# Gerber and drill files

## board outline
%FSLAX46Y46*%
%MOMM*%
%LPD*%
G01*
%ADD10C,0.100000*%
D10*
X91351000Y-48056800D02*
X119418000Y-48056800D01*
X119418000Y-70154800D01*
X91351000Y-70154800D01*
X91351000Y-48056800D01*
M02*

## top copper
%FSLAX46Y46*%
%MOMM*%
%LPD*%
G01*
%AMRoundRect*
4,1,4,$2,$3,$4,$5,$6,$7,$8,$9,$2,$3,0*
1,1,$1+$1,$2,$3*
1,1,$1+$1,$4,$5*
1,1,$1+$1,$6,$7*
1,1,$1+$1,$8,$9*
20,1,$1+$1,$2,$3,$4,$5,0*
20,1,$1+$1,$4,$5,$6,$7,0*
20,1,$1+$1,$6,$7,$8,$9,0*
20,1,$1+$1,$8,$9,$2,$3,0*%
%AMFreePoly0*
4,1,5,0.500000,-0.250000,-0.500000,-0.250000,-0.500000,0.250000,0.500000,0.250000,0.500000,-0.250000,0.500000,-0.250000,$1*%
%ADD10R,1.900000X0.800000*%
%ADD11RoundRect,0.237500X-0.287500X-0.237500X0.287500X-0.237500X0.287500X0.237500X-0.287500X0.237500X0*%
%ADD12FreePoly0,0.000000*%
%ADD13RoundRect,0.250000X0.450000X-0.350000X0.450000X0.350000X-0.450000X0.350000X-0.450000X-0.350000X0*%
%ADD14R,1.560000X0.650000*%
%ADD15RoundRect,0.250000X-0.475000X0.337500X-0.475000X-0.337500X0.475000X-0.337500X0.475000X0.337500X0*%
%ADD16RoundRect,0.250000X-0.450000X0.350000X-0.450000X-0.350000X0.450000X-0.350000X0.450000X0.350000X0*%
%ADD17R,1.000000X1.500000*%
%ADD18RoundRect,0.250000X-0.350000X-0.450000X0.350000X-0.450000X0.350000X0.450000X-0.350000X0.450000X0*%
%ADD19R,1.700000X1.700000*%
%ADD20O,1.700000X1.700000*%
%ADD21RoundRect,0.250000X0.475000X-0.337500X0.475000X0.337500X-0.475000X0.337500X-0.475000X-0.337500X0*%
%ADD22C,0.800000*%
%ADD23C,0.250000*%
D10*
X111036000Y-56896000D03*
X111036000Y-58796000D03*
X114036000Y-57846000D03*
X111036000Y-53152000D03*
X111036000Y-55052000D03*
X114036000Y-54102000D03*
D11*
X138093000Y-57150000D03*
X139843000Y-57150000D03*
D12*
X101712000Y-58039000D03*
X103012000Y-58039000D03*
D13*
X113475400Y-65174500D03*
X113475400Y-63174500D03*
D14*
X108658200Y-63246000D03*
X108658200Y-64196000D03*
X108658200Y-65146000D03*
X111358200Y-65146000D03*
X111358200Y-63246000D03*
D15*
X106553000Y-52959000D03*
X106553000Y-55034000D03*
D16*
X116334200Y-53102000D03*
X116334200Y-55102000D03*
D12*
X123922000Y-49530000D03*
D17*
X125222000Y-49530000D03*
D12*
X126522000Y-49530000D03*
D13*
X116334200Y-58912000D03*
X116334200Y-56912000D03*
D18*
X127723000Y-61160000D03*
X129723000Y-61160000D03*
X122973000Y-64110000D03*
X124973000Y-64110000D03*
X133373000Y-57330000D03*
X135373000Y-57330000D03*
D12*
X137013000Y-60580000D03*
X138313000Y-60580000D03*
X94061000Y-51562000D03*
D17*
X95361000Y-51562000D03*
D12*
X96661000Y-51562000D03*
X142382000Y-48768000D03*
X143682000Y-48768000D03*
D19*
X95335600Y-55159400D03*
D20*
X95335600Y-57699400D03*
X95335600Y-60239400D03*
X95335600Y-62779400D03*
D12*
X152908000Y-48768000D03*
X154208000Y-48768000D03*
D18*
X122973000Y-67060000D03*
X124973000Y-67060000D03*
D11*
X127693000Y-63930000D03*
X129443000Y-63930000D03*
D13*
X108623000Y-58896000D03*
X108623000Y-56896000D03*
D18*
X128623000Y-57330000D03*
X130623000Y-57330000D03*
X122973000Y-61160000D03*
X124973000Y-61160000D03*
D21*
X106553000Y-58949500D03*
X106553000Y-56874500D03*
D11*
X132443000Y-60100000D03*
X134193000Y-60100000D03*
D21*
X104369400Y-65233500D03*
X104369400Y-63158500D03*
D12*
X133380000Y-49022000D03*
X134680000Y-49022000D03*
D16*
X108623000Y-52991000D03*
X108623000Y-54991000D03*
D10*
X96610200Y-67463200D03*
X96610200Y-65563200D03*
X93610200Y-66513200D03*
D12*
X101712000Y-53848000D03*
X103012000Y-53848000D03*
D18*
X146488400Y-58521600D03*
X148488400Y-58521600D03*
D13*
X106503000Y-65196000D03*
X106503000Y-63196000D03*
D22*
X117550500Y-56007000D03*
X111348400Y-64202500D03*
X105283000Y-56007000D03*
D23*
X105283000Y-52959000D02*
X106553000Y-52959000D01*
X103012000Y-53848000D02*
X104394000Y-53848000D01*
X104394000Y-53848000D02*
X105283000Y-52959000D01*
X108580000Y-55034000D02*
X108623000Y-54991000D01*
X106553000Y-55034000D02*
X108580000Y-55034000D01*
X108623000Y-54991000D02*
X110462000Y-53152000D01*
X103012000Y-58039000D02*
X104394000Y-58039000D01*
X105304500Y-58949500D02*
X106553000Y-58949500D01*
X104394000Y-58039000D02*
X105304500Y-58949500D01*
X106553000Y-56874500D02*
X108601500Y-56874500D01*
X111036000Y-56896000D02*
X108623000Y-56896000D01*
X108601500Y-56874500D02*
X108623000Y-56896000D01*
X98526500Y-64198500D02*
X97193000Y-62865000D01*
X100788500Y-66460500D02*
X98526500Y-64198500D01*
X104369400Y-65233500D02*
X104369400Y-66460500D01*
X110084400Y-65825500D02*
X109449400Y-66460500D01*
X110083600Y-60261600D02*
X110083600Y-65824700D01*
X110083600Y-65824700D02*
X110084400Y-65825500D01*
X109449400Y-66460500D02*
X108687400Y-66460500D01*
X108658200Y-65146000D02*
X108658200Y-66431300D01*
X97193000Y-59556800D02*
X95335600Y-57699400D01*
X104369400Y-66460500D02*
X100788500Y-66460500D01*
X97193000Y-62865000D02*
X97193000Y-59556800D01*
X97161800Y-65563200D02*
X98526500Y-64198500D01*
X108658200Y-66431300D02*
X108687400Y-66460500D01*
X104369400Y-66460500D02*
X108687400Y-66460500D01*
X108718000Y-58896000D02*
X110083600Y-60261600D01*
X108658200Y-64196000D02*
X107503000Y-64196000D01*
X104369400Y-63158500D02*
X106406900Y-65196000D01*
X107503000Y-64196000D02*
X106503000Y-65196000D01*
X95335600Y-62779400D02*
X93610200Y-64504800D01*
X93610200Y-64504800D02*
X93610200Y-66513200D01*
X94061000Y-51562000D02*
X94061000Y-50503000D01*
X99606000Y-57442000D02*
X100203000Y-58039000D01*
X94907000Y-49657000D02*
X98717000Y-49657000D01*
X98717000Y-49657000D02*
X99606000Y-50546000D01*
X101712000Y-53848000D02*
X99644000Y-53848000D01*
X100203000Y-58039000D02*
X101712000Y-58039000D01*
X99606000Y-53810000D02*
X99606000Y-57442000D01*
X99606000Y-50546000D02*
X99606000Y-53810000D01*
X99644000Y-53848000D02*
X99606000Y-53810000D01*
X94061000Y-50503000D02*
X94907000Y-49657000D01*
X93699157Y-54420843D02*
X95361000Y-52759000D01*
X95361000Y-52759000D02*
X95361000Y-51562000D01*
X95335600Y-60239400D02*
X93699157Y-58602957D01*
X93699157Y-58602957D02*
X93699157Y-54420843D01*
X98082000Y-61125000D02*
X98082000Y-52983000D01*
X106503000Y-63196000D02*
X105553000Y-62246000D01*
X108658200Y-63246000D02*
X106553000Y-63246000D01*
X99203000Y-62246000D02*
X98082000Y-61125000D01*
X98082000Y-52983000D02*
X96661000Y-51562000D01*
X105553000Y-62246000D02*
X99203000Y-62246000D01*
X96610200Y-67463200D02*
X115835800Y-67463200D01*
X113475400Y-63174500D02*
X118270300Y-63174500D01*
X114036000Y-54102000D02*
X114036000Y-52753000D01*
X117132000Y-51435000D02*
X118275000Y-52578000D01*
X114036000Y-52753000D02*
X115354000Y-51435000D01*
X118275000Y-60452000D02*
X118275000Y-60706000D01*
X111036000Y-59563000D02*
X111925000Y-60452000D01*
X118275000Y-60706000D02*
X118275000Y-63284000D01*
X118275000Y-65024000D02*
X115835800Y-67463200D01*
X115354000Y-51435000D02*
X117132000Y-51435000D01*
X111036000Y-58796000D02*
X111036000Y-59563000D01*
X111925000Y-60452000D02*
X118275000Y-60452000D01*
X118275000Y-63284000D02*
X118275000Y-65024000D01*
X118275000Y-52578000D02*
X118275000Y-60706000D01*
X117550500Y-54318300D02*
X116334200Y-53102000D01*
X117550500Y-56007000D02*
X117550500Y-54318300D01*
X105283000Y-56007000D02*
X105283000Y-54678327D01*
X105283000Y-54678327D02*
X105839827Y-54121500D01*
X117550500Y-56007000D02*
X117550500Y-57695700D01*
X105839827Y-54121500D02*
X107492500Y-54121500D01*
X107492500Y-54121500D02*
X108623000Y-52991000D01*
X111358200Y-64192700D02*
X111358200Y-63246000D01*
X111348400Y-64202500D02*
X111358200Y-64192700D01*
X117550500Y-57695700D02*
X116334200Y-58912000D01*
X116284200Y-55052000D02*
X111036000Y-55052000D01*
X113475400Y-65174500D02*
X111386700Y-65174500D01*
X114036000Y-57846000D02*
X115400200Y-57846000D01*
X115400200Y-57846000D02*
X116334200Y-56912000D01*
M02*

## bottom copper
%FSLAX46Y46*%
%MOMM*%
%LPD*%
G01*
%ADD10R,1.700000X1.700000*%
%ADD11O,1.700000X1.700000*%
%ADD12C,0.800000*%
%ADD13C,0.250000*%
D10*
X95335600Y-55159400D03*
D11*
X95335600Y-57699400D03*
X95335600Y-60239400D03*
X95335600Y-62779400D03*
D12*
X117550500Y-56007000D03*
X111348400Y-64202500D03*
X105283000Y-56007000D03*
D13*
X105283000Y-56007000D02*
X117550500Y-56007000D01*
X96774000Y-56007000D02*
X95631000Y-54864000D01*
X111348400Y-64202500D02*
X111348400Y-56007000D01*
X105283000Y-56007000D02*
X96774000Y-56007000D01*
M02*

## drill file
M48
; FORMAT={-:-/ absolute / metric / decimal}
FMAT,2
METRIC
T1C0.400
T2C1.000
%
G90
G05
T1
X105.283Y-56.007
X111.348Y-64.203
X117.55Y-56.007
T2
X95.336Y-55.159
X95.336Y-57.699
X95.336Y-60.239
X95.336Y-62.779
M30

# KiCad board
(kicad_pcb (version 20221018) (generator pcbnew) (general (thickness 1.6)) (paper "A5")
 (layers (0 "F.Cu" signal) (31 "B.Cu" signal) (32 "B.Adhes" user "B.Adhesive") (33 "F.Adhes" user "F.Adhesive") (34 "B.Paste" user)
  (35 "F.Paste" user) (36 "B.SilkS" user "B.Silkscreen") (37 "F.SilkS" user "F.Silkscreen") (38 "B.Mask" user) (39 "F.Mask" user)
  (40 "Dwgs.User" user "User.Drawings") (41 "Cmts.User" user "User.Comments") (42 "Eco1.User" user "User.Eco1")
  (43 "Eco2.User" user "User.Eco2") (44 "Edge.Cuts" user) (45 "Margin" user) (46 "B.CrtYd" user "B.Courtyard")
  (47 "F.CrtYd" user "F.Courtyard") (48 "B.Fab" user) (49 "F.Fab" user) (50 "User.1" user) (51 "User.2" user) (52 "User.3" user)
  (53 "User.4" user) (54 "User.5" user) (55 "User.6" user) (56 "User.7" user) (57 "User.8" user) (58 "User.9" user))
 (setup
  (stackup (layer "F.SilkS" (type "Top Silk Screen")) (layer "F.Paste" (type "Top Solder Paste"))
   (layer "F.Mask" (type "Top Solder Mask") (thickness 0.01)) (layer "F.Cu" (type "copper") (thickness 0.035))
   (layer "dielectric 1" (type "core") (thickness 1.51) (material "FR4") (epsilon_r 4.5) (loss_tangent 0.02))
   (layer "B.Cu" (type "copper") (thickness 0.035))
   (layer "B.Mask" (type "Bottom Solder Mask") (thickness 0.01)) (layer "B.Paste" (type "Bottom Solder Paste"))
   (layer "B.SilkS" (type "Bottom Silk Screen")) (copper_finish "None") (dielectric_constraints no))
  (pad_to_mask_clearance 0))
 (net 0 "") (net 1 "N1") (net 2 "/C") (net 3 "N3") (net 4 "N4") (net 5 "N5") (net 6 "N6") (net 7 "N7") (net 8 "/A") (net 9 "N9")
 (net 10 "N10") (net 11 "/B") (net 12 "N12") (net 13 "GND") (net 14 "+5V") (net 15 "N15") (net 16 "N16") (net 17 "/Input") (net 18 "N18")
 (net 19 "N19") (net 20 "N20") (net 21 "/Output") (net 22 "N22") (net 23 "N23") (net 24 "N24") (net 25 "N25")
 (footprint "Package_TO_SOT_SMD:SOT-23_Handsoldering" (layer "F.Cu") (at 112.536 57.846)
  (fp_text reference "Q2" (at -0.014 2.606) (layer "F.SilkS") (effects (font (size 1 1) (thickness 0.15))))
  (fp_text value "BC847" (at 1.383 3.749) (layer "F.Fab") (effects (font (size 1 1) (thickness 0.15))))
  (pad "1" smd rect (at -1.5 -0.95) (size 1.9 0.8) (layers "F.Cu" "F.Paste" "F.Mask") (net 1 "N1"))
  (pad "2" smd rect (at -1.5 0.95) (size 1.9 0.8) (layers "F.Cu" "F.Paste" "F.Mask") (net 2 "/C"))
  (pad "3" smd rect (at 1.5 0) (size 1.9 0.8) (layers "F.Cu" "F.Paste" "F.Mask") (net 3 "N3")))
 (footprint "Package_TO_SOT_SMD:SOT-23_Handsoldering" (layer "F.Cu") (at 112.536 54.102)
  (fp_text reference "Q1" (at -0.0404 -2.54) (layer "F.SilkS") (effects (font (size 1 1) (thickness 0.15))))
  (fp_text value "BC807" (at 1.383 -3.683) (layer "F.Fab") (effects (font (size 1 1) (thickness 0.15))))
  (pad "1" smd rect (at -1.5 -0.95) (size 1.9 0.8) (layers "F.Cu" "F.Paste" "F.Mask") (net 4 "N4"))
  (pad "2" smd rect (at -1.5 0.95) (size 1.9 0.8) (layers "F.Cu" "F.Paste" "F.Mask") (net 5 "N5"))
  (pad "3" smd rect (at 1.5 0) (size 1.9 0.8) (layers "F.Cu" "F.Paste" "F.Mask") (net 2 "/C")))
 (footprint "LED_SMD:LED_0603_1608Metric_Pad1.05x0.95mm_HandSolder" (layer "F.Cu") (at 138.968 57.15)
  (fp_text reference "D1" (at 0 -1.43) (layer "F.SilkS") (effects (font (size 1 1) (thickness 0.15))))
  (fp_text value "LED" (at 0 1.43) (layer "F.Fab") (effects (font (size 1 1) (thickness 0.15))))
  (pad "1" smd roundrect (at -0.875 0) (size 1.05 0.95) (layers "F.Cu" "F.Paste" "F.Mask") (roundrect_rratio 0.25) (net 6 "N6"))
  (pad "2" smd roundrect (at 0.875 0) (size 1.05 0.95) (layers "F.Cu" "F.Paste" "F.Mask") (roundrect_rratio 0.25) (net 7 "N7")))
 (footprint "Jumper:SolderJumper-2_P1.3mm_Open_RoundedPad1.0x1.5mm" (layer "F.Cu") (at 102.362 58.039)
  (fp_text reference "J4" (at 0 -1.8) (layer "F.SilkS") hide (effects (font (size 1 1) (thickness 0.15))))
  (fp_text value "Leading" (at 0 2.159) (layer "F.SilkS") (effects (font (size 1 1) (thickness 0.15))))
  (pad "1" smd custom (at -0.65 0) (size 1 0.5) (layers "F.Cu" "F.Mask") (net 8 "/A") (zone_connect 2) (thermal_bridge_angle 45)
   (options (clearance outline) (anchor rect)) (primitives))
  (pad "2" smd custom (at 0.65 0) (size 1 0.5) (layers "F.Cu" "F.Mask") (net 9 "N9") (zone_connect 2) (thermal_bridge_angle 45)
   (options (clearance outline) (anchor rect)) (primitives)))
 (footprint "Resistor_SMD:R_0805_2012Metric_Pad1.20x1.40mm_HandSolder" (layer "F.Cu") (at 113.4754 64.1745 90)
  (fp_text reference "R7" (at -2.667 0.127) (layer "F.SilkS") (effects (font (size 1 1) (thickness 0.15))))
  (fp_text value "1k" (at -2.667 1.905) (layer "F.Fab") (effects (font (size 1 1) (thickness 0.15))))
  (pad "1" smd roundrect (at -1 0 90) (size 1.2 1.4) (layers "F.Cu" "F.Paste" "F.Mask") (roundrect_rratio 0.208333) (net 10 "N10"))
  (pad "2" smd roundrect (at 1 0 90) (size 1.2 1.4) (layers "F.Cu" "F.Paste" "F.Mask") (roundrect_rratio 0.208333) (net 2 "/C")))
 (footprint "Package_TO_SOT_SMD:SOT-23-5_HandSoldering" (layer "F.Cu") (at 110.0082 64.196)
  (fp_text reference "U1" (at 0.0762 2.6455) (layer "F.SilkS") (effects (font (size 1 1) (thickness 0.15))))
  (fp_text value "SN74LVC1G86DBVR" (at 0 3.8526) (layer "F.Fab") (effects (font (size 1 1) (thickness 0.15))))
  (pad "1" smd rect (at -1.35 -0.95) (size 1.56 0.65) (layers "F.Cu" "F.Paste" "F.Mask") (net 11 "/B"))
  (pad "2" smd rect (at -1.35 0) (size 1.56 0.65) (layers "F.Cu" "F.Paste" "F.Mask") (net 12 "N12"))
  (pad "3" smd rect (at -1.35 0.95) (size 1.56 0.65) (layers "F.Cu" "F.Paste" "F.Mask") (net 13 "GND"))
  (pad "4" smd rect (at 1.35 0.95) (size 1.56 0.65) (layers "F.Cu" "F.Paste" "F.Mask") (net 10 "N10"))
  (pad "5" smd rect (at 1.35 -0.95) (size 1.56 0.65) (layers "F.Cu" "F.Paste" "F.Mask") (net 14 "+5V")))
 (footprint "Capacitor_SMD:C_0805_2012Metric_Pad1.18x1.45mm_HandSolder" (layer "F.Cu") (at 106.553 53.9965 -90)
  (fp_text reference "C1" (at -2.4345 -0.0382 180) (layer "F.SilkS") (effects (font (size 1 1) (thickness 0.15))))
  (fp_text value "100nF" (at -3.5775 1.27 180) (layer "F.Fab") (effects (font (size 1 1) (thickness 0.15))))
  (pad "1" smd roundrect (at -1.0375 0 270) (size 1.175 1.45) (layers "F.Cu" "F.Paste" "F.Mask") (roundrect_rratio 0.2127659574)
   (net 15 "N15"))
  (pad "2" smd roundrect (at 1.0375 0 270) (size 1.175 1.45) (layers "F.Cu" "F.Paste" "F.Mask") (roundrect_rratio 0.2127659574) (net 4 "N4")))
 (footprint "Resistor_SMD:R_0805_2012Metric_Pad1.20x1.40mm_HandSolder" (layer "F.Cu") (at 116.3342 54.102 -90)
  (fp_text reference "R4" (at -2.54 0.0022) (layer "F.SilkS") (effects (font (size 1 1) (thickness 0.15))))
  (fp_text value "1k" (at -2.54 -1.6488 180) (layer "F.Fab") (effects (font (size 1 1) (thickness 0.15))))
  (pad "1" smd roundrect (at -1 0 270) (size 1.2 1.4) (layers "F.Cu" "F.Paste" "F.Mask") (roundrect_rratio 0.2083333333) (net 14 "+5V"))
  (pad "2" smd roundrect (at 1 0 270) (size 1.2 1.4) (layers "F.Cu" "F.Paste" "F.Mask") (roundrect_rratio 0.2083333333) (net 5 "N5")))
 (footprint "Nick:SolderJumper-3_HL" (layer "F.Cu") (at 125.222 49.53)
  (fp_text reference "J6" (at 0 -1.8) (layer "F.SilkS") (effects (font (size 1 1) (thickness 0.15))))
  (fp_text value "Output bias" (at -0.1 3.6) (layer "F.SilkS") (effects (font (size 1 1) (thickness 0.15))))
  (pad "1" smd custom (at -1.3 0) (size 1 0.5) (layers "F.Cu" "F.Mask") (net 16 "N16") (zone_connect 2) (thermal_bridge_angle 45)
   (options (clearance outline) (anchor rect)) (primitives))
  (pad "2" smd rect (at 0 0) (size 1 1.5) (layers "F.Cu" "F.Mask") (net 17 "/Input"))
  (pad "3" smd custom (at 1.3 0) (size 1 0.5) (layers "F.Cu" "F.Mask") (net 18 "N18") (zone_connect 2) (thermal_bridge_angle 45)
   (options (clearance outline) (anchor rect)) (primitives)))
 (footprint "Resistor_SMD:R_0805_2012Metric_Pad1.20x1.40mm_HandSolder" (layer "F.Cu") (at 116.3342 57.912 90)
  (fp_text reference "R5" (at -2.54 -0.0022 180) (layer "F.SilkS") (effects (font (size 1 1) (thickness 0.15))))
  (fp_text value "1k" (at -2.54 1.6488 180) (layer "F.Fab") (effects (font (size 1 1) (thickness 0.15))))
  (pad "1" smd roundrect (at -1 0 90) (size 1.2 1.4) (layers "F.Cu" "F.Paste" "F.Mask") (roundrect_rratio 0.2083333333) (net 14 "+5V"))
  (pad "2" smd roundrect (at 1 0 90) (size 1.2 1.4) (layers "F.Cu" "F.Paste" "F.Mask") (roundrect_rratio 0.2083333333) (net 3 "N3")))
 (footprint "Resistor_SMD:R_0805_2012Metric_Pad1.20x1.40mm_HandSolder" (layer "F.Cu") (at 128.723 61.16)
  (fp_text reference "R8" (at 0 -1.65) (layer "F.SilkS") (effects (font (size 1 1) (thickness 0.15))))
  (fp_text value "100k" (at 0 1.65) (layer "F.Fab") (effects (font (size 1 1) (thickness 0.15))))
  (pad "1" smd roundrect (at -1 0) (size 1.2 1.4) (layers "F.Cu" "F.Paste" "F.Mask") (roundrect_rratio 0.208333) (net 16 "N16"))
  (pad "2" smd roundrect (at 1 0) (size 1.2 1.4) (layers "F.Cu" "F.Paste" "F.Mask") (roundrect_rratio 0.208333) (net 14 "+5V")))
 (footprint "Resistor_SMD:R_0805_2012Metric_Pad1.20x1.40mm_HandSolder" (layer "F.Cu") (at 123.973 64.11)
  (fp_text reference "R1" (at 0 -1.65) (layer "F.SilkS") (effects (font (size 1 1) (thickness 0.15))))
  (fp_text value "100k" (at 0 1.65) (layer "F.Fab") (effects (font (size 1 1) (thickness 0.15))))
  (pad "1" smd roundrect (at -1 0) (size 1.2 1.4) (layers "F.Cu" "F.Paste" "F.Mask") (roundrect_rratio 0.208333) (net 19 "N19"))
  (pad "2" smd roundrect (at 1 0) (size 1.2 1.4) (layers "F.Cu" "F.Paste" "F.Mask") (roundrect_rratio 0.208333) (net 14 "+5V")))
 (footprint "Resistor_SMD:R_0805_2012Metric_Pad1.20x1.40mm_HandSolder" (layer "F.Cu") (at 134.373 57.33)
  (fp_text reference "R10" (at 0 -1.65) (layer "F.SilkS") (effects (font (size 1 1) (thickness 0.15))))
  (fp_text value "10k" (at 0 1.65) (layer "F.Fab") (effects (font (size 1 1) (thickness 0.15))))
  (pad "1" smd roundrect (at -1 0) (size 1.2 1.4) (layers "F.Cu" "F.Paste" "F.Mask") (roundrect_rratio 0.208333) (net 13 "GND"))
  (pad "2" smd roundrect (at 1 0) (size 1.2 1.4) (layers "F.Cu" "F.Paste" "F.Mask") (roundrect_rratio 0.208333) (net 6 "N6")))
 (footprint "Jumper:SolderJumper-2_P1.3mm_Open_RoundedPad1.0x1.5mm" (layer "F.Cu") (at 137.663 60.58)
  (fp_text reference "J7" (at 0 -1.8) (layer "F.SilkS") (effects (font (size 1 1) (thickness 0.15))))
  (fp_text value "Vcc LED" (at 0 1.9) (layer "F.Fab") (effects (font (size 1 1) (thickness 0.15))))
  (pad "1" smd custom (at -0.65 0) (size 1 0.5) (layers "F.Cu" "F.Mask") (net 7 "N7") (zone_connect 2) (thermal_bridge_angle 45)
   (options (clearance outline) (anchor rect)) (primitives))
  (pad "2" smd custom (at 0.65 0) (size 1 0.5) (layers "F.Cu" "F.Mask") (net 14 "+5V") (zone_connect 2) (thermal_bridge_angle 45)
   (options (clearance outline) (anchor rect)) (primitives)))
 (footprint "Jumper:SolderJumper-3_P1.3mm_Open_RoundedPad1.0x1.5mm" (layer "F.Cu") (at 95.361 51.562)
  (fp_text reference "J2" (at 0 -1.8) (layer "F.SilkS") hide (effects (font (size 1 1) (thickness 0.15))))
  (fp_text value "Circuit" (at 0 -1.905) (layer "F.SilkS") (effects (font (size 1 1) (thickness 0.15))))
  (pad "1" smd custom (at -1.3 0) (size 1 0.5) (layers "F.Cu" "F.Mask") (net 8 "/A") (zone_connect 2) (thermal_bridge_angle 45)
   (options (clearance outline) (anchor rect)) (primitives))
  (pad "2" smd rect (at 0 0) (size 1 1.5) (layers "F.Cu" "F.Mask") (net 17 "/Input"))
  (pad "3" smd custom (at 1.3 0) (size 1 0.5) (layers "F.Cu" "F.Mask") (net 11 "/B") (zone_connect 2) (thermal_bridge_angle 45)
   (options (clearance outline) (anchor rect)) (primitives)))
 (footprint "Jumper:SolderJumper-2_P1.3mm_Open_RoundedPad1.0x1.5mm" (layer "F.Cu") (at 143.032 48.768)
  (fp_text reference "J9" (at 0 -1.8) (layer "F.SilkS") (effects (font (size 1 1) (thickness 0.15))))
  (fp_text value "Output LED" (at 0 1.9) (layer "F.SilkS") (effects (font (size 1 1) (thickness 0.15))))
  (pad "1" smd custom (at -0.65 0) (size 1 0.5) (layers "F.Cu" "F.Mask") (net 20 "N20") (zone_connect 2) (thermal_bridge_angle 45)
   (options (clearance outline) (anchor rect)) (primitives))
  (pad "2" smd custom (at 0.65 0) (size 1 0.5) (layers "F.Cu" "F.Mask") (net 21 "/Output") (zone_connect 2) (thermal_bridge_angle 45)
   (options (clearance outline) (anchor rect)) (primitives)))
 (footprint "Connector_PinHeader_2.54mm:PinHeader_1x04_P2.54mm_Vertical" (layer "F.Cu") (at 95.3356 55.1594)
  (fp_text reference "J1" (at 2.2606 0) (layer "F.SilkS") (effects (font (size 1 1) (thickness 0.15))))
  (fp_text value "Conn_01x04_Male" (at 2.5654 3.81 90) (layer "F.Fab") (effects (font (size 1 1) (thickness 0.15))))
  (pad "1" thru_hole rect (at 0 0) (size 1.7 1.7) (drill 1) (layers "*.Cu" "*.Mask") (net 14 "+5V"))
  (pad "2" thru_hole oval (at 0 2.54) (size 1.7 1.7) (drill 1) (layers "*.Cu" "*.Mask") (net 13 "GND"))
  (pad "3" thru_hole oval (at 0 5.08) (size 1.7 1.7) (drill 1) (layers "*.Cu" "*.Mask") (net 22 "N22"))
  (pad "4" thru_hole oval (at 0 7.62) (size 1.7 1.7) (drill 1) (layers "*.Cu" "*.Mask") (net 21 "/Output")))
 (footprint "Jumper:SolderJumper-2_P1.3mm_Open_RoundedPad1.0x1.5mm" (layer "F.Cu") (at 153.558 48.768)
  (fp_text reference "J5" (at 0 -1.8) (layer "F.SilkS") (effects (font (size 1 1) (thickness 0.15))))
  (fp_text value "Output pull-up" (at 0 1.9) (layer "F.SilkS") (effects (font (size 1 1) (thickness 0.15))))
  (pad "1" smd custom (at -0.65 0) (size 1 0.5) (layers "F.Cu" "F.Mask") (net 21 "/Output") (zone_connect 2) (thermal_bridge_angle 45)
   (options (clearance outline) (anchor rect)) (primitives))
  (pad "2" smd custom (at 0.65 0) (size 1 0.5) (layers "F.Cu" "F.Mask") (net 19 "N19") (zone_connect 2) (thermal_bridge_angle 45)
   (options (clearance outline) (anchor rect)) (primitives)))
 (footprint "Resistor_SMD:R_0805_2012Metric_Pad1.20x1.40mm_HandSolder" (layer "F.Cu") (at 123.973 67.06)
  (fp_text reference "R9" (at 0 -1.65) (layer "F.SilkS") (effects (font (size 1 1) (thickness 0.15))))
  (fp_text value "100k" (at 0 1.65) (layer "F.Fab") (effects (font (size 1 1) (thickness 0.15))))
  (pad "1" smd roundrect (at -1 0) (size 1.2 1.4) (layers "F.Cu" "F.Paste" "F.Mask") (roundrect_rratio 0.208333) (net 13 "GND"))
  (pad "2" smd roundrect (at 1 0) (size 1.2 1.4) (layers "F.Cu" "F.Paste" "F.Mask") (roundrect_rratio 0.208333) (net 18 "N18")))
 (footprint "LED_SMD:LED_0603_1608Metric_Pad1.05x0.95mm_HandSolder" (layer "F.Cu") (at 128.568 63.93)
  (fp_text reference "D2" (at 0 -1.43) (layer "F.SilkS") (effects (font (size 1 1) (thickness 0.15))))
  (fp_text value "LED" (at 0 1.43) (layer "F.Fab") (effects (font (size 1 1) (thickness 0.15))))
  (pad "1" smd roundrect (at -0.875 0) (size 1.05 0.95) (layers "F.Cu" "F.Paste" "F.Mask") (roundrect_rratio 0.25) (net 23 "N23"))
  (pad "2" smd roundrect (at 0.875 0) (size 1.05 0.95) (layers "F.Cu" "F.Paste" "F.Mask") (roundrect_rratio 0.25) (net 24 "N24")))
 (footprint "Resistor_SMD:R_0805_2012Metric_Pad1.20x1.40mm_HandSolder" (layer "F.Cu") (at 108.623 57.896 90)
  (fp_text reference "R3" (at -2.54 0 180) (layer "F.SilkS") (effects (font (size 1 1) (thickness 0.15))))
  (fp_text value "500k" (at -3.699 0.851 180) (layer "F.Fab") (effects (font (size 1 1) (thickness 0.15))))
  (pad "1" smd roundrect (at -1 0 90) (size 1.2 1.4) (layers "F.Cu" "F.Paste" "F.Mask") (roundrect_rratio 0.2083333333) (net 13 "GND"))
  (pad "2" smd roundrect (at 1 0 90) (size 1.2 1.4) (layers "F.Cu" "F.Paste" "F.Mask") (roundrect_rratio 0.2083333333) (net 1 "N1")))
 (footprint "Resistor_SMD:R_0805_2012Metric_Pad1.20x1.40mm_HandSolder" (layer "F.Cu") (at 129.623 57.33)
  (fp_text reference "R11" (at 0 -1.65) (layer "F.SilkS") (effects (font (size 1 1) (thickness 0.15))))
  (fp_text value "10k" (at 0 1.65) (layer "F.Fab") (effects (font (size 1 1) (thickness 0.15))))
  (pad "1" smd roundrect (at -1 0) (size 1.2 1.4) (layers "F.Cu" "F.Paste" "F.Mask") (roundrect_rratio 0.208333) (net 13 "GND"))
  (pad "2" smd roundrect (at 1 0) (size 1.2 1.4) (layers "F.Cu" "F.Paste" "F.Mask") (roundrect_rratio 0.208333) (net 23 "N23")))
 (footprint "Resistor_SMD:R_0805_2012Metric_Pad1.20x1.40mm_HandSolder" (layer "F.Cu") (at 123.973 61.16)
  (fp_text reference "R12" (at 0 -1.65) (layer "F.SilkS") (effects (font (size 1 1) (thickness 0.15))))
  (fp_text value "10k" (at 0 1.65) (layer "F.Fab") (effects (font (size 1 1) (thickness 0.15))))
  (pad "1" smd roundrect (at -1 0) (size 1.2 1.4) (layers "F.Cu" "F.Paste" "F.Mask") (roundrect_rratio 0.208333) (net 13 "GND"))
  (pad "2" smd roundrect (at 1 0) (size 1.2 1.4) (layers "F.Cu" "F.Paste" "F.Mask") (roundrect_rratio 0.208333) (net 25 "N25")))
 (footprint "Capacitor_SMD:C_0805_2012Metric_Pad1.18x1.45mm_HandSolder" (layer "F.Cu") (at 106.553 57.912 90)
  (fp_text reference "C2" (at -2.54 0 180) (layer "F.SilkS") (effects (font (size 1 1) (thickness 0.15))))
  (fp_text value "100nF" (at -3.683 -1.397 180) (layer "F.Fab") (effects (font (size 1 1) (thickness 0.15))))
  (pad "1" smd roundrect (at -1.0375 0 90) (size 1.175 1.45) (layers "F.Cu" "F.Paste" "F.Mask") (roundrect_rratio 0.2127659574) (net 9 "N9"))
  (pad "2" smd roundrect (at 1.0375 0 90) (size 1.175 1.45) (layers "F.Cu" "F.Paste" "F.Mask") (roundrect_rratio 0.2127659574) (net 1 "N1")))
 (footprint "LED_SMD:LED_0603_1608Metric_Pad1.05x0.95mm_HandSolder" (layer "F.Cu") (at 133.318 60.1)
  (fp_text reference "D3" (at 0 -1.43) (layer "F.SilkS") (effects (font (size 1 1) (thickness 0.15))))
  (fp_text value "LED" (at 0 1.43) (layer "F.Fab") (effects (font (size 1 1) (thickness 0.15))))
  (pad "1" smd roundrect (at -0.875 0) (size 1.05 0.95) (layers "F.Cu" "F.Paste" "F.Mask") (roundrect_rratio 0.25) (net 25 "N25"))
  (pad "2" smd roundrect (at 0.875 0) (size 1.05 0.95) (layers "F.Cu" "F.Paste" "F.Mask") (roundrect_rratio 0.25) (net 20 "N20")))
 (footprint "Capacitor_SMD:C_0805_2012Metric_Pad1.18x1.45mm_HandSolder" (layer "F.Cu") (at 104.3694 64.196 90)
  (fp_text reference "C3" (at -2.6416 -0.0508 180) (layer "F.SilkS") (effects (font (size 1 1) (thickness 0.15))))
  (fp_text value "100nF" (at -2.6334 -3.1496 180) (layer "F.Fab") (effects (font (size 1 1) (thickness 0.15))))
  (pad "1" smd roundrect (at -1.0375 0 90) (size 1.175 1.45) (layers "F.Cu" "F.Paste" "F.Mask") (roundrect_rratio 0.2127659574)
   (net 13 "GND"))
  (pad "2" smd roundrect (at 1.0375 0 90) (size 1.175 1.45) (layers "F.Cu" "F.Paste" "F.Mask") (roundrect_rratio 0.2127659574)
   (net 12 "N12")))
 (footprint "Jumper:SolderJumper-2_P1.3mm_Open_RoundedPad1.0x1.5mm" (layer "F.Cu") (at 134.03 49.022)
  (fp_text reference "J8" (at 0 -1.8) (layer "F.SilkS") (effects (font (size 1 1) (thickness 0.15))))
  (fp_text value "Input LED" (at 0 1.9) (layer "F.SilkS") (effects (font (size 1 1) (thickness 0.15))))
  (pad "1" smd custom (at -0.65 0) (size 1 0.5) (layers "F.Cu" "F.Mask") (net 24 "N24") (zone_connect 2) (thermal_bridge_angle 45)
   (options (clearance outline) (anchor rect)) (primitives))
  (pad "2" smd custom (at 0.65 0) (size 1 0.5) (layers "F.Cu" "F.Mask") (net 17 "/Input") (zone_connect 2) (thermal_bridge_angle 45)
   (options (clearance outline) (anchor rect)) (primitives)))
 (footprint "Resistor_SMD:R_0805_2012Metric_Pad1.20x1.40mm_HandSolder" (layer "F.Cu") (at 108.623 53.991 -90)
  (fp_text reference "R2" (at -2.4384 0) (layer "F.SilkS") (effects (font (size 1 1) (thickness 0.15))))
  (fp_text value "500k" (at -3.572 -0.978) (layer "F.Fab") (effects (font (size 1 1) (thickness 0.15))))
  (pad "1" smd roundrect (at -1 0 270) (size 1.2 1.4) (layers "F.Cu" "F.Paste" "F.Mask") (roundrect_rratio 0.2083333333) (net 14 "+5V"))
  (pad "2" smd roundrect (at 1 0 270) (size 1.2 1.4) (layers "F.Cu" "F.Paste" "F.Mask") (roundrect_rratio 0.2083333333) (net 4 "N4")))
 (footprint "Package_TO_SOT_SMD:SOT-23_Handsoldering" (layer "F.Cu") (at 95.1102 66.5132 180)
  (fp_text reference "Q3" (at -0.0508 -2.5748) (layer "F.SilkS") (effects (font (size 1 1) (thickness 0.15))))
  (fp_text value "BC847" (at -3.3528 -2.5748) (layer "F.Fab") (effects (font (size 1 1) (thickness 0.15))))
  (pad "1" smd rect (at -1.5 -0.95 180) (size 1.9 0.8) (layers "F.Cu" "F.Paste" "F.Mask") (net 2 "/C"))
  (pad "2" smd rect (at -1.5 0.95 180) (size 1.9 0.8) (layers "F.Cu" "F.Paste" "F.Mask") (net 13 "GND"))
  (pad "3" smd rect (at 1.5 0 180) (size 1.9 0.8) (layers "F.Cu" "F.Paste" "F.Mask") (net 21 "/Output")))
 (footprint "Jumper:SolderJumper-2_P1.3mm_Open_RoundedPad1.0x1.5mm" (layer "F.Cu") (at 102.362 53.848)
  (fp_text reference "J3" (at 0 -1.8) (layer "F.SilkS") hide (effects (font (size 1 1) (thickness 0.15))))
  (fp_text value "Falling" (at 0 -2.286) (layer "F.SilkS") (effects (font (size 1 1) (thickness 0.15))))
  (pad "1" smd custom (at -0.65 0) (size 1 0.5) (layers "F.Cu" "F.Mask") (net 8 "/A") (zone_connect 2) (thermal_bridge_angle 45)
   (options (clearance outline) (anchor rect)) (primitives))
  (pad "2" smd custom (at 0.65 0) (size 1 0.5) (layers "F.Cu" "F.Mask") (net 15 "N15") (zone_connect 2) (thermal_bridge_angle 45)
   (options (clearance outline) (anchor rect)) (primitives)))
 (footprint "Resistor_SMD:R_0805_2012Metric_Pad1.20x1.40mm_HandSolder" (layer "F.Cu") (at 147.4884 58.5216)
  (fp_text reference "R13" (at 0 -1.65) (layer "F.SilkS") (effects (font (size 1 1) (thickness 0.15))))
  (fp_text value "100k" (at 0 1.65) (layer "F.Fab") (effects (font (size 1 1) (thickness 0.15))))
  (pad "1" smd roundrect (at -1 0) (size 1.2 1.4) (layers "F.Cu" "F.Paste" "F.Mask") (roundrect_rratio 0.208333) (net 17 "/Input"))
  (pad "2" smd roundrect (at 1 0) (size 1.2 1.4) (layers "F.Cu" "F.Paste" "F.Mask") (roundrect_rratio 0.208333) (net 22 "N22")))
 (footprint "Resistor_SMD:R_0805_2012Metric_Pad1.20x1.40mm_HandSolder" (layer "F.Cu") (at 106.503 64.196 90)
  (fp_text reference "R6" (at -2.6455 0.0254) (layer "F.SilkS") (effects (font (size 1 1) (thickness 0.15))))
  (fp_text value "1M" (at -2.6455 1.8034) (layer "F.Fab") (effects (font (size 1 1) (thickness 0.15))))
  (pad "1" smd roundrect (at -1 0 90) (size 1.2 1.4) (layers "F.Cu" "F.Paste" "F.Mask") (roundrect_rratio 0.2083333333) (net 12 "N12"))
  (pad "2" smd roundrect (at 1 0 90) (size 1.2 1.4) (layers "F.Cu" "F.Paste" "F.Mask") (roundrect_rratio 0.2083333333) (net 11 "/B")))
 (gr_rect (start 91.351 48.0568) (end 119.418 70.1548) (stroke (width 0.1) (type solid)) (fill none) (layer "Edge.Cuts"))
 (segment (start 105.283 52.959) (end 106.553 52.959) (width 0.25) (layer "F.Cu") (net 15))
 (segment (start 103.012 53.848) (end 104.394 53.848) (width 0.25) (layer "F.Cu") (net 15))
 (segment (start 104.394 53.848) (end 105.283 52.959) (width 0.25) (layer "F.Cu") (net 15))
 (segment (start 108.58 55.034) (end 108.623 54.991) (width 0.25) (layer "F.Cu") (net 4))
 (segment (start 106.553 55.034) (end 108.58 55.034) (width 0.25) (layer "F.Cu") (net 4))
 (segment (start 108.623 54.991) (end 110.462 53.152) (width 0.25) (layer "F.Cu") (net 4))
 (segment (start 103.012 58.039) (end 104.394 58.039) (width 0.25) (layer "F.Cu") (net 9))
 (segment (start 105.3045 58.9495) (end 106.553 58.9495) (width 0.25) (layer "F.Cu") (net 9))
 (segment (start 104.394 58.039) (end 105.3045 58.9495) (width 0.25) (layer "F.Cu") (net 9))
 (segment (start 106.553 56.8745) (end 108.6015 56.8745) (width 0.25) (layer "F.Cu") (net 1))
 (segment (start 111.036 56.896) (end 108.623 56.896) (width 0.25) (layer "F.Cu") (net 1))
 (segment (start 108.6015 56.8745) (end 108.623 56.896) (width 0.25) (layer "F.Cu") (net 1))
 (segment (start 98.5265 64.1985) (end 97.193 62.865) (width 0.25) (layer "F.Cu") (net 13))
 (segment (start 100.7885 66.4605) (end 98.5265 64.1985) (width 0.25) (layer "F.Cu") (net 13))
 (segment (start 104.3694 65.2335) (end 104.3694 66.4605) (width 0.25) (layer "F.Cu") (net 13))
 (segment (start 110.0844 65.8255) (end 109.4494 66.4605) (width 0.25) (layer "F.Cu") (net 13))
 (segment (start 110.0836 60.2616) (end 110.0836 65.8247) (width 0.25) (layer "F.Cu") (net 13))
 (segment (start 110.0836 65.8247) (end 110.0844 65.8255) (width 0.25) (layer "F.Cu") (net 13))
 (segment (start 109.4494 66.4605) (end 108.6874 66.4605) (width 0.25) (layer "F.Cu") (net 13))
 (segment (start 108.6582 65.146) (end 108.6582 66.4313) (width 0.25) (layer "F.Cu") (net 13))
 (segment (start 97.193 59.5568) (end 95.3356 57.6994) (width 0.25) (layer "F.Cu") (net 13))
 (segment (start 104.3694 66.4605) (end 100.7885 66.4605) (width 0.25) (layer "F.Cu") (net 13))
 (segment (start 97.193 62.865) (end 97.193 59.5568) (width 0.25) (layer "F.Cu") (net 13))
 (segment (start 97.1618 65.5632) (end 98.5265 64.1985) (width 0.25) (layer "F.Cu") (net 13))
 (segment (start 108.6582 66.4313) (end 108.6874 66.4605) (width 0.25) (layer "F.Cu") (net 13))
 (segment (start 104.3694 66.4605) (end 108.6874 66.4605) (width 0.25) (layer "F.Cu") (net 13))
 (segment (start 108.718 58.896) (end 110.0836 60.2616) (width 0.25) (layer "F.Cu") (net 13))
 (segment (start 108.6582 64.196) (end 107.503 64.196) (width 0.25) (layer "F.Cu") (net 12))
 (segment (start 104.3694 63.1585) (end 106.4069 65.196) (width 0.25) (layer "F.Cu") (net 12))
 (segment (start 107.503 64.196) (end 106.503 65.196) (width 0.25) (layer "F.Cu") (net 12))
 (segment (start 95.3356 62.7794) (end 93.6102 64.5048) (width 0.25) (layer "F.Cu") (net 21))
 (segment (start 93.6102 64.5048) (end 93.6102 66.5132) (width 0.25) (layer "F.Cu") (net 21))
 (segment (start 94.061 51.562) (end 94.061 50.503) (width 0.25) (layer "F.Cu") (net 8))
 (segment (start 99.606 57.442) (end 100.203 58.039) (width 0.25) (layer "F.Cu") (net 8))
 (segment (start 94.907 49.657) (end 98.717 49.657) (width 0.25) (layer "F.Cu") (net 8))
 (segment (start 98.717 49.657) (end 99.606 50.546) (width 0.25) (layer "F.Cu") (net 8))
 (segment (start 101.712 53.848) (end 99.644 53.848) (width 0.25) (layer "F.Cu") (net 8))
 (segment (start 100.203 58.039) (end 101.712 58.039) (width 0.25) (layer "F.Cu") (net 8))
 (segment (start 99.606 53.81) (end 99.606 57.442) (width 0.25) (layer "F.Cu") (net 8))
 (segment (start 99.606 50.546) (end 99.606 53.81) (width 0.25) (layer "F.Cu") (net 8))
 (segment (start 99.644 53.848) (end 99.606 53.81) (width 0.25) (layer "F.Cu") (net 8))
 (segment (start 94.061 50.503) (end 94.907 49.657) (width 0.25) (layer "F.Cu") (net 8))
 (segment (start 93.699157 54.420843) (end 95.361 52.759) (width 0.25) (layer "F.Cu") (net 17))
 (segment (start 95.361 52.759) (end 95.361 51.562) (width 0.25) (layer "F.Cu") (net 17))
 (segment (start 95.3356 60.2394) (end 93.699157 58.602957) (width 0.25) (layer "F.Cu") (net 17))
 (segment (start 93.699157 58.602957) (end 93.699157 54.420843) (width 0.25) (layer "F.Cu") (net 17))
 (segment (start 98.082 61.125) (end 98.082 52.983) (width 0.25) (layer "F.Cu") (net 11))
 (segment (start 106.503 63.196) (end 105.553 62.246) (width 0.25) (layer "F.Cu") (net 11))
 (segment (start 108.6582 63.246) (end 106.553 63.246) (width 0.25) (layer "F.Cu") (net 11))
 (segment (start 99.203 62.246) (end 98.082 61.125) (width 0.25) (layer "F.Cu") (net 11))
 (segment (start 98.082 52.983) (end 96.661 51.562) (width 0.25) (layer "F.Cu") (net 11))
 (segment (start 105.553 62.246) (end 99.203 62.246) (width 0.25) (layer "F.Cu") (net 11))
 (segment (start 96.6102 67.4632) (end 115.8358 67.4632) (width 0.25) (layer "F.Cu") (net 2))
 (segment (start 113.4754 63.1745) (end 118.2703 63.1745) (width 0.25) (layer "F.Cu") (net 2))
 (segment (start 114.036 54.102) (end 114.036 52.753) (width 0.25) (layer "F.Cu") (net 2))
 (segment (start 117.132 51.435) (end 118.275 52.578) (width 0.25) (layer "F.Cu") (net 2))
 (segment (start 114.036 52.753) (end 115.354 51.435) (width 0.25) (layer "F.Cu") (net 2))
 (segment (start 118.275 60.452) (end 118.275 60.706) (width 0.25) (layer "F.Cu") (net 2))
 (segment (start 111.036 59.563) (end 111.925 60.452) (width 0.25) (layer "F.Cu") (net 2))
 (segment (start 118.275 60.706) (end 118.275 63.284) (width 0.25) (layer "F.Cu") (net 2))
 (segment (start 118.275 65.024) (end 115.8358 67.4632) (width 0.25) (layer "F.Cu") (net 2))
 (segment (start 115.354 51.435) (end 117.132 51.435) (width 0.25) (layer "F.Cu") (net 2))
 (segment (start 111.036 58.796) (end 111.036 59.563) (width 0.25) (layer "F.Cu") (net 2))
 (segment (start 111.925 60.452) (end 118.275 60.452) (width 0.25) (layer "F.Cu") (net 2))
 (segment (start 118.275 63.284) (end 118.275 65.024) (width 0.25) (layer "F.Cu") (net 2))
 (segment (start 118.275 52.578) (end 118.275 60.706) (width 0.25) (layer "F.Cu") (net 2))
 (segment (start 117.5505 54.3183) (end 116.3342 53.102) (width 0.25) (layer "F.Cu") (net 14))
 (segment (start 117.5505 56.007) (end 117.5505 54.3183) (width 0.25) (layer "F.Cu") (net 14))
 (segment (start 105.283 56.007) (end 105.283 54.678327) (width 0.25) (layer "F.Cu") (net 14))
 (segment (start 105.283 54.678327) (end 105.839827 54.1215) (width 0.25) (layer "F.Cu") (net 14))
 (segment (start 117.5505 56.007) (end 117.5505 57.6957) (width 0.25) (layer "F.Cu") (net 14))
 (segment (start 105.839827 54.1215) (end 107.4925 54.1215) (width 0.25) (layer "F.Cu") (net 14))
 (segment (start 107.4925 54.1215) (end 108.623 52.991) (width 0.25) (layer "F.Cu") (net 14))
 (segment (start 111.3582 64.1927) (end 111.3582 63.246) (width 0.25) (layer "F.Cu") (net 14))
 (segment (start 111.3484 64.2025) (end 111.3582 64.1927) (width 0.25) (layer "F.Cu") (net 14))
 (segment (start 117.5505 57.6957) (end 116.3342 58.912) (width 0.25) (layer "F.Cu") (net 14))
 (via (at 117.5505 56.007) (size 0.8) (drill 0.4) (layers "F.Cu" "B.Cu") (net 14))
 (via (at 111.3484 64.2025) (size 0.8) (drill 0.4) (layers "F.Cu" "B.Cu") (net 14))
 (via (at 105.283 56.007) (size 0.8) (drill 0.4) (layers "F.Cu" "B.Cu") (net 14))
 (segment (start 105.283 56.007) (end 117.5505 56.007) (width 0.25) (layer "B.Cu") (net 14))
 (segment (start 96.774 56.007) (end 95.631 54.864) (width 0.25) (layer "B.Cu") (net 14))
 (segment (start 111.3484 64.2025) (end 111.3484 56.007) (width 0.25) (layer "B.Cu") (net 14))
 (segment (start 105.283 56.007) (end 96.774 56.007) (width 0.25) (layer "B.Cu") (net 14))
 (segment (start 116.2842 55.052) (end 111.036 55.052) (width 0.25) (layer "F.Cu") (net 5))
 (segment (start 113.4754 65.1745) (end 111.3867 65.1745) (width 0.25) (layer "F.Cu") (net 10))
 (segment (start 114.036 57.846) (end 115.4002 57.846) (width 0.25) (layer "F.Cu") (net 3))
 (segment (start 115.4002 57.846) (end 116.3342 56.912) (width 0.25) (layer "F.Cu") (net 3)))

